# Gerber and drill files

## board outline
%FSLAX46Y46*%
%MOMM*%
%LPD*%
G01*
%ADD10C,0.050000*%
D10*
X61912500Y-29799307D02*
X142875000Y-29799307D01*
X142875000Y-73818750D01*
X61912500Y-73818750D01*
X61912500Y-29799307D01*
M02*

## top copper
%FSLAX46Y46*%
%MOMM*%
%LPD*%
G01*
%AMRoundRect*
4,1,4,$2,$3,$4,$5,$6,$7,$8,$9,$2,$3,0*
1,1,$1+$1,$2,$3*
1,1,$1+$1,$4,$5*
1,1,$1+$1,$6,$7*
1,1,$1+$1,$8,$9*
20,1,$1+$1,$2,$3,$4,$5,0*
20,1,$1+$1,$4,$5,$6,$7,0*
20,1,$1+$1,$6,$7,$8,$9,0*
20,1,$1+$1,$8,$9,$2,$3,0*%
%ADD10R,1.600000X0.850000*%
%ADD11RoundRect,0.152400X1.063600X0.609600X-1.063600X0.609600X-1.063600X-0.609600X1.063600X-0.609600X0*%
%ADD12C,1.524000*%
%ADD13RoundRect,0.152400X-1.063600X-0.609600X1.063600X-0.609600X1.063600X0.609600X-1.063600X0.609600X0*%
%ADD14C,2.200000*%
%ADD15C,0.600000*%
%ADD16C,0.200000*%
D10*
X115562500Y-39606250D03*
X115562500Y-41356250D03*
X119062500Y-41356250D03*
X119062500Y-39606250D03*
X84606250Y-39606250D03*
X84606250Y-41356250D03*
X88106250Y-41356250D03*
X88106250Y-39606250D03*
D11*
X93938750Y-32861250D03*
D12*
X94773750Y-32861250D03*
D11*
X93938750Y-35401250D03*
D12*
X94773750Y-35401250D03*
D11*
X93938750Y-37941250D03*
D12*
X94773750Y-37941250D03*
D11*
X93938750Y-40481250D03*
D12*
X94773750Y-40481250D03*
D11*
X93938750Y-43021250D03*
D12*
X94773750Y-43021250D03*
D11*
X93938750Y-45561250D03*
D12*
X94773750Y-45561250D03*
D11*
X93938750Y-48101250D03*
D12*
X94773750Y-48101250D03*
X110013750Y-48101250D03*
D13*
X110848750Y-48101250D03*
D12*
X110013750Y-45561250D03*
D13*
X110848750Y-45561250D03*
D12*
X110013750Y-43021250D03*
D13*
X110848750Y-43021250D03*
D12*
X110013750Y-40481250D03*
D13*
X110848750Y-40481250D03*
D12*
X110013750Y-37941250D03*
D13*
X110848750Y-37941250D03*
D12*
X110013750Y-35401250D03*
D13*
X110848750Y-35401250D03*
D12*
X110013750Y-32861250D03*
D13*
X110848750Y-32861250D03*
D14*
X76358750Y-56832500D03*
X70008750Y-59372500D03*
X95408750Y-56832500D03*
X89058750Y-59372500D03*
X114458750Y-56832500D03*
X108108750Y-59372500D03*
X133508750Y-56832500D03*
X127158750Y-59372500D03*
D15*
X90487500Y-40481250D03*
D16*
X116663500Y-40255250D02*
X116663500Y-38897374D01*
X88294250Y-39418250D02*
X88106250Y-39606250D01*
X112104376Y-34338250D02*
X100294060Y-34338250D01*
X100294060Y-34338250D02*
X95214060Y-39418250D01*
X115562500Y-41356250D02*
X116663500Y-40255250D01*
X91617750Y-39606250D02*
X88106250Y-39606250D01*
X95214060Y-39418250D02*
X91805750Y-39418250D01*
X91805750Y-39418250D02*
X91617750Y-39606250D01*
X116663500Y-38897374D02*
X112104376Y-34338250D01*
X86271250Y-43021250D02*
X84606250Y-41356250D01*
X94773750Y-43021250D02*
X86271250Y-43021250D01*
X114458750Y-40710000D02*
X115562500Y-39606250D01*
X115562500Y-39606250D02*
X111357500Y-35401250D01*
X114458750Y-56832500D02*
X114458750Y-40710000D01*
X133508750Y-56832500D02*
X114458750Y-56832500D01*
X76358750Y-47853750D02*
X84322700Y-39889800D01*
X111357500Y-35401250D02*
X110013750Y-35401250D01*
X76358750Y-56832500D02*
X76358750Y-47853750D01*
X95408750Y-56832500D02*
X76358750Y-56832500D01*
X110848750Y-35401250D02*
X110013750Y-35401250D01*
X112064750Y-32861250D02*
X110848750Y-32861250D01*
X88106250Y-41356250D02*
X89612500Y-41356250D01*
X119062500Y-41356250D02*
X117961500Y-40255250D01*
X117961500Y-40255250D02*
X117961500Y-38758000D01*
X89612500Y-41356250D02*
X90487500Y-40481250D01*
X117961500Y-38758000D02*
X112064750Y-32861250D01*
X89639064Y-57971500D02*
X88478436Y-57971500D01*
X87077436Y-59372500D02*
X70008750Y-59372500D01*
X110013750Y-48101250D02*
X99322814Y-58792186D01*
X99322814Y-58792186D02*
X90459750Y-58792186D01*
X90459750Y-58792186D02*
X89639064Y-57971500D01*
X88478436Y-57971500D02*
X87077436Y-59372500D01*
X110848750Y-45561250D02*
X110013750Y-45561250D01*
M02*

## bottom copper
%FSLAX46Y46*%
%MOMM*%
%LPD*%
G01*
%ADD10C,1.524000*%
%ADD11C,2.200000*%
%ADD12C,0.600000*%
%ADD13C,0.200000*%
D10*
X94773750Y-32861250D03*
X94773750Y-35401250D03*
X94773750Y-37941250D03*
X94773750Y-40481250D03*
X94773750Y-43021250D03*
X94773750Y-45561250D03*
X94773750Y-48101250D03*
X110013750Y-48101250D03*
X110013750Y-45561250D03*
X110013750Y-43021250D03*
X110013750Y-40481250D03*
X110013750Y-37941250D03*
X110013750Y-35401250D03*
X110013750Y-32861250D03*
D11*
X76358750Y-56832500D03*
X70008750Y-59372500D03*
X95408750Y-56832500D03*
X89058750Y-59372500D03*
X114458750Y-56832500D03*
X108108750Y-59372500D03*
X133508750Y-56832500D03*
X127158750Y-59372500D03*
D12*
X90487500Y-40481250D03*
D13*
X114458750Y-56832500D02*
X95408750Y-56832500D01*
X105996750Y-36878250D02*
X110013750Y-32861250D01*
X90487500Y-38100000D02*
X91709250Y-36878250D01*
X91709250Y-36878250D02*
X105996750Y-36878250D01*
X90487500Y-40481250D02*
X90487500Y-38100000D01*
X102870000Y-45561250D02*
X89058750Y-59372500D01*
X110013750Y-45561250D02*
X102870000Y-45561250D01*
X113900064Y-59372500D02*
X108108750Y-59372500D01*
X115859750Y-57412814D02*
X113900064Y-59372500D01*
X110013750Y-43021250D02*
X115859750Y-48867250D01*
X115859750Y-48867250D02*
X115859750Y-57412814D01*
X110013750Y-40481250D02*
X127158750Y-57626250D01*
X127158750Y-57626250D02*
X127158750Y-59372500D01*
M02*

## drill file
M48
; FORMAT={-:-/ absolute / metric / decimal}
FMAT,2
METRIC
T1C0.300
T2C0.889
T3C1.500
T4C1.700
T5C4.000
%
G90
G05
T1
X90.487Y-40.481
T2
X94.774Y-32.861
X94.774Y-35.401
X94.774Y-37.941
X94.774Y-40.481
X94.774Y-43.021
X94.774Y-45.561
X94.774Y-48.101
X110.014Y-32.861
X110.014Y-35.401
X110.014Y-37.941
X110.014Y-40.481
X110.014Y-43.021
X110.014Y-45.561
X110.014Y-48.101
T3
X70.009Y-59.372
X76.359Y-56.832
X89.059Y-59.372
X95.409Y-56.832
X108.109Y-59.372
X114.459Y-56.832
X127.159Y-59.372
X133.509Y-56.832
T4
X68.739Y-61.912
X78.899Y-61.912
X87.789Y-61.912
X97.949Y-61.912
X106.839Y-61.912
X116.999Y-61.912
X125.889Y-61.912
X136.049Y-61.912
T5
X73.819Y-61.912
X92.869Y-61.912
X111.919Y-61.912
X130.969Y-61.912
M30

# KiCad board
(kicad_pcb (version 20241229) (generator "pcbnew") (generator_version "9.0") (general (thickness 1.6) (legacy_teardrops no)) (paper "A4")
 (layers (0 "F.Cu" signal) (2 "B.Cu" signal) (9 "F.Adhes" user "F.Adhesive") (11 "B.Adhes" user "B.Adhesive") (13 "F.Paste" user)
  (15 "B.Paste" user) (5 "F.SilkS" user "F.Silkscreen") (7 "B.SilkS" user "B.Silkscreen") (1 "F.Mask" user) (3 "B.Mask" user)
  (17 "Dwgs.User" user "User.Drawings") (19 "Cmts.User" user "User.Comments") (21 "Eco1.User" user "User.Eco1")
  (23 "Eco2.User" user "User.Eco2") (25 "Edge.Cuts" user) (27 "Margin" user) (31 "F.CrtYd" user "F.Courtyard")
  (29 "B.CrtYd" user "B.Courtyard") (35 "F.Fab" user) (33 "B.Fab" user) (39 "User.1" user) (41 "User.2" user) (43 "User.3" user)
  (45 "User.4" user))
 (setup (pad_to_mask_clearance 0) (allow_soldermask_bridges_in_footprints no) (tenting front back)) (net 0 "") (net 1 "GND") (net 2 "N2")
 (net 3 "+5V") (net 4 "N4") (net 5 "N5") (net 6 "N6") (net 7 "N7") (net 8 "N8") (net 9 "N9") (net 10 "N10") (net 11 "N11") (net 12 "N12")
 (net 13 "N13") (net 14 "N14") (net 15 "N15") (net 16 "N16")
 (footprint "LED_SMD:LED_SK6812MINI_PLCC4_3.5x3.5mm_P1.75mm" (layer "F.Cu") (at 117.3125 40.48125)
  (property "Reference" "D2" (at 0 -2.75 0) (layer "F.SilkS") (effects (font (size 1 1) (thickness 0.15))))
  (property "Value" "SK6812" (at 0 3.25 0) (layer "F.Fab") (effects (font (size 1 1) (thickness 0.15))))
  (pad "1" smd rect (at -1.75 -0.875) (size 1.6 0.85) (layers "F.Cu" "F.Mask" "F.Paste") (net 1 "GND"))
  (pad "2" smd rect (at -1.75 0.875) (size 1.6 0.85) (layers "F.Cu" "F.Mask" "F.Paste") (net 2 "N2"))
  (pad "3" smd rect (at 1.75 0.875) (size 1.6 0.85) (layers "F.Cu" "F.Mask" "F.Paste") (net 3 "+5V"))
  (pad "4" smd rect (at 1.75 -0.875) (size 1.6 0.85) (layers "F.Cu" "F.Mask" "F.Paste") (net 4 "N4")))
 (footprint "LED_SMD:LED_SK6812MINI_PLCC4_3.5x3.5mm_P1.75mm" (layer "F.Cu") (at 86.35625 40.48125)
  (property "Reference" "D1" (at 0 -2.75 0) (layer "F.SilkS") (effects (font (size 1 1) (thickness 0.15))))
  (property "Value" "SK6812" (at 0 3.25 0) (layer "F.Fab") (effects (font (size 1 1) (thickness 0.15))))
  (pad "1" smd rect (at -1.75 -0.875) (size 1.6 0.85) (layers "F.Cu" "F.Mask" "F.Paste") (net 1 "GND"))
  (pad "2" smd rect (at -1.75 0.875) (size 1.6 0.85) (layers "F.Cu" "F.Mask" "F.Paste") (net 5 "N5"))
  (pad "3" smd rect (at 1.75 0.875) (size 1.6 0.85) (layers "F.Cu" "F.Mask" "F.Paste") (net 3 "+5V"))
  (pad "4" smd rect (at 1.75 -0.875) (size 1.6 0.85) (layers "F.Cu" "F.Mask" "F.Paste") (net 2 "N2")))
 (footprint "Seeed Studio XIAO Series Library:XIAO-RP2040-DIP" (layer "F.Cu") (at 102.39375 40.48125)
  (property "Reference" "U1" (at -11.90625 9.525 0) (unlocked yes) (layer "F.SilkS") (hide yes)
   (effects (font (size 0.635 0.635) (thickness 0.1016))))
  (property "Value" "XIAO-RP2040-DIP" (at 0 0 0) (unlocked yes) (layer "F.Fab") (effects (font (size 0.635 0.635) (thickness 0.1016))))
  (pad "1" smd roundrect (at -8.455 -7.62 180) (size 2.432 1.524) (layers "F.Cu" "F.Mask") (roundrect_rratio 0.1) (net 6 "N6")
   (thermal_bridge_angle 45))
  (pad "1" thru_hole circle (at -7.62 -7.62 180) (size 1.524 1.524) (drill 0.889) (layers "*.Cu" "*.Mask") (remove_unused_layers no)
   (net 6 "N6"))
  (pad "2" smd roundrect (at -8.455 -5.08 180) (size 2.432 1.524) (layers "F.Cu" "F.Mask") (roundrect_rratio 0.1) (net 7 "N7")
   (thermal_bridge_angle 45))
  (pad "2" thru_hole circle (at -7.62 -5.08 180) (size 1.524 1.524) (drill 0.889) (layers "*.Cu" "*.Mask") (remove_unused_layers no)
   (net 7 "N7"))
  (pad "3" smd roundrect (at -8.455 -2.54 180) (size 2.432 1.524) (layers "F.Cu" "F.Mask") (roundrect_rratio 0.1) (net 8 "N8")
   (thermal_bridge_angle 45))
  (pad "3" thru_hole circle (at -7.62 -2.54 180) (size 1.524 1.524) (drill 0.889) (layers "*.Cu" "*.Mask") (remove_unused_layers no)
   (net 8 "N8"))
  (pad "4" smd roundrect (at -8.455 0 180) (size 2.432 1.524) (layers "F.Cu" "F.Mask") (roundrect_rratio 0.1) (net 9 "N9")
   (thermal_bridge_angle 45))
  (pad "4" thru_hole circle (at -7.62 0 180) (size 1.524 1.524) (drill 0.889) (layers "*.Cu" "*.Mask") (remove_unused_layers no)
   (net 9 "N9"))
  (pad "5" smd roundrect (at -8.455 2.54 180) (size 2.432 1.524) (layers "F.Cu" "F.Mask") (roundrect_rratio 0.1) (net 5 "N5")
   (thermal_bridge_angle 45))
  (pad "5" thru_hole circle (at -7.62 2.54 180) (size 1.524 1.524) (drill 0.889) (layers "*.Cu" "*.Mask") (remove_unused_layers no)
   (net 5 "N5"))
  (pad "6" smd roundrect (at -8.455 5.08 180) (size 2.432 1.524) (layers "F.Cu" "F.Mask") (roundrect_rratio 0.1) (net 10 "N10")
   (thermal_bridge_angle 45))
  (pad "6" thru_hole circle (at -7.62 5.08 180) (size 1.524 1.524) (drill 0.889) (layers "*.Cu" "*.Mask") (remove_unused_layers no)
   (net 10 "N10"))
  (pad "7" smd roundrect (at -8.455 7.62 180) (size 2.432 1.524) (layers "F.Cu" "F.Mask") (roundrect_rratio 0.1) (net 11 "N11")
   (thermal_bridge_angle 45))
  (pad "7" thru_hole circle (at -7.62 7.62 180) (size 1.524 1.524) (drill 0.889) (layers "*.Cu" "*.Mask") (remove_unused_layers no)
   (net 11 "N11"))
  (pad "8" thru_hole circle (at 7.62 7.62) (size 1.524 1.524) (drill 0.889) (layers "*.Cu" "*.Mask") (remove_unused_layers no)
   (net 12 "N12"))
  (pad "8" smd roundrect (at 8.455 7.62) (size 2.432 1.524) (layers "F.Cu" "F.Mask") (roundrect_rratio 0.1) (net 12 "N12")
   (thermal_bridge_angle 45))
  (pad "9" thru_hole circle (at 7.62 5.08) (size 1.524 1.524) (drill 0.889) (layers "*.Cu" "*.Mask") (remove_unused_layers no)
   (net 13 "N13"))
  (pad "9" smd roundrect (at 8.455 5.08) (size 2.432 1.524) (layers "F.Cu" "F.Mask") (roundrect_rratio 0.1) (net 13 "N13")
   (thermal_bridge_angle 45))
  (pad "10" thru_hole circle (at 7.62 2.54) (size 1.524 1.524) (drill 0.889) (layers "*.Cu" "*.Mask") (remove_unused_layers no)
   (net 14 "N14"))
  (pad "10" smd roundrect (at 8.455 2.54) (size 2.432 1.524) (layers "F.Cu" "F.Mask") (roundrect_rratio 0.1) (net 14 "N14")
   (thermal_bridge_angle 45))
  (pad "11" thru_hole circle (at 7.62 0) (size 1.524 1.524) (drill 0.889) (layers "*.Cu" "*.Mask") (remove_unused_layers no) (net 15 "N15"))
  (pad "11" smd roundrect (at 8.455 0) (size 2.432 1.524) (layers "F.Cu" "F.Mask") (roundrect_rratio 0.1) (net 15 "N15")
   (thermal_bridge_angle 45))
  (pad "12" thru_hole circle (at 7.62 -2.54) (size 1.524 1.524) (drill 0.889) (layers "*.Cu" "*.Mask") (remove_unused_layers no)
   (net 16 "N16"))
  (pad "12" smd roundrect (at 8.455 -2.54) (size 2.432 1.524) (layers "F.Cu" "F.Mask") (roundrect_rratio 0.1) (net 16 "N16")
   (thermal_bridge_angle 45))
  (pad "13" thru_hole circle (at 7.62 -5.08) (size 1.524 1.524) (drill 0.889) (layers "*.Cu" "*.Mask") (remove_unused_layers no)
   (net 1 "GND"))
  (pad "13" smd roundrect (at 8.455 -5.08) (size 2.432 1.524) (layers "F.Cu" "F.Mask") (roundrect_rratio 0.1) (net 1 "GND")
   (thermal_bridge_angle 45))
  (pad "14" thru_hole circle (at 7.62 -7.62) (size 1.524 1.524) (drill 0.889) (layers "*.Cu" "*.Mask") (remove_unused_layers no)
   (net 3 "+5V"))
  (pad "14" smd roundrect (at 8.455 -7.62) (size 2.432 1.524) (layers "F.Cu" "F.Mask") (roundrect_rratio 0.1) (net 3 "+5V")
   (thermal_bridge_angle 45)))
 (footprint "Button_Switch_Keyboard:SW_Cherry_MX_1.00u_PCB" (layer "F.Cu") (at 76.35875 56.8325)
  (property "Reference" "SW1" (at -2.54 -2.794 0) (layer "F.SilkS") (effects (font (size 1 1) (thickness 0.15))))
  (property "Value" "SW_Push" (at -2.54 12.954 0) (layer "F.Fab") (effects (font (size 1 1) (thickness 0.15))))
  (pad "" np_thru_hole circle (at -7.62 5.08) (size 1.7 1.7) (drill 1.7) (layers "*.Cu" "*.Mask"))
  (pad "" np_thru_hole circle (at -2.54 5.08) (size 4 4) (drill 4) (layers "*.Cu" "*.Mask"))
  (pad "" np_thru_hole circle (at 2.54 5.08) (size 1.7 1.7) (drill 1.7) (layers "*.Cu" "*.Mask"))
  (pad "1" thru_hole circle (at 0 0) (size 2.2 2.2) (drill 1.5) (layers "*.Cu" "*.Mask") (remove_unused_layers no) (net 1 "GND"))
  (pad "2" thru_hole circle (at -6.35 2.54) (size 2.2 2.2) (drill 1.5) (layers "*.Cu" "*.Mask") (remove_unused_layers no) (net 12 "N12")))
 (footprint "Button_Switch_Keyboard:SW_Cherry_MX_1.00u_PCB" (layer "F.Cu") (at 95.40875 56.8325)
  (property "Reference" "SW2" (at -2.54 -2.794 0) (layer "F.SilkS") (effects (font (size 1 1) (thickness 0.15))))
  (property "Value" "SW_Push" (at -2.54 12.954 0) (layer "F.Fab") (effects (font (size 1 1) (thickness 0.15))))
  (pad "" np_thru_hole circle (at -7.62 5.08) (size 1.7 1.7) (drill 1.7) (layers "*.Cu" "*.Mask"))
  (pad "" np_thru_hole circle (at -2.54 5.08) (size 4 4) (drill 4) (layers "*.Cu" "*.Mask"))
  (pad "" np_thru_hole circle (at 2.54 5.08) (size 1.7 1.7) (drill 1.7) (layers "*.Cu" "*.Mask"))
  (pad "1" thru_hole circle (at 0 0) (size 2.2 2.2) (drill 1.5) (layers "*.Cu" "*.Mask") (remove_unused_layers no) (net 1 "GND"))
  (pad "2" thru_hole circle (at -6.35 2.54) (size 2.2 2.2) (drill 1.5) (layers "*.Cu" "*.Mask") (remove_unused_layers no) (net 13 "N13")))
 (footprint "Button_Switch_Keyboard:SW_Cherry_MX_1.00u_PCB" (layer "F.Cu") (at 114.45875 56.8325)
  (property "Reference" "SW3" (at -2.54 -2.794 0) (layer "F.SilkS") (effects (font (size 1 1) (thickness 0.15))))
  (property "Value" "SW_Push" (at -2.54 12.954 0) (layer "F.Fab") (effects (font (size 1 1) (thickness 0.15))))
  (pad "" np_thru_hole circle (at -7.62 5.08) (size 1.7 1.7) (drill 1.7) (layers "*.Cu" "*.Mask"))
  (pad "" np_thru_hole circle (at -2.54 5.08) (size 4 4) (drill 4) (layers "*.Cu" "*.Mask"))
  (pad "" np_thru_hole circle (at 2.54 5.08) (size 1.7 1.7) (drill 1.7) (layers "*.Cu" "*.Mask"))
  (pad "1" thru_hole circle (at 0 0) (size 2.2 2.2) (drill 1.5) (layers "*.Cu" "*.Mask") (remove_unused_layers no) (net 1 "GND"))
  (pad "2" thru_hole circle (at -6.35 2.54) (size 2.2 2.2) (drill 1.5) (layers "*.Cu" "*.Mask") (remove_unused_layers no) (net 14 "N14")))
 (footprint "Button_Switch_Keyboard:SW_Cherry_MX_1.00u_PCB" (layer "F.Cu") (at 133.50875 56.8325)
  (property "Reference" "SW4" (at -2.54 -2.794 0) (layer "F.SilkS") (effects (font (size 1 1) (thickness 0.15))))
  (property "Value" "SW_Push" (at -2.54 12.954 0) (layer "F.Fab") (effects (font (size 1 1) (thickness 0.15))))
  (pad "" np_thru_hole circle (at -7.62 5.08) (size 1.7 1.7) (drill 1.7) (layers "*.Cu" "*.Mask"))
  (pad "" np_thru_hole circle (at -2.54 5.08) (size 4 4) (drill 4) (layers "*.Cu" "*.Mask"))
  (pad "" np_thru_hole circle (at 2.54 5.08) (size 1.7 1.7) (drill 1.7) (layers "*.Cu" "*.Mask"))
  (pad "1" thru_hole circle (at 0 0) (size 2.2 2.2) (drill 1.5) (layers "*.Cu" "*.Mask") (remove_unused_layers no) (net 1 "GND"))
  (pad "2" thru_hole circle (at -6.35 2.54) (size 2.2 2.2) (drill 1.5) (layers "*.Cu" "*.Mask") (remove_unused_layers no) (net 15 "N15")))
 (gr_rect (start 61.9125 29.799307) (end 142.875 73.81875) (stroke (width 0.05) (type default)) (fill no) (layer "Edge.Cuts"))
 (segment (start 116.6635 40.25525) (end 116.6635 38.897374) (width 0.2) (layer "F.Cu") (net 2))
 (segment (start 88.29425 39.41825) (end 88.10625 39.60625) (width 0.2) (layer "F.Cu") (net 2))
 (segment (start 112.104376 34.33825) (end 100.29406 34.33825) (width 0.2) (layer "F.Cu") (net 2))
 (segment (start 100.29406 34.33825) (end 95.21406 39.41825) (width 0.2) (layer "F.Cu") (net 2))
 (segment (start 115.5625 41.35625) (end 116.6635 40.25525) (width 0.2) (layer "F.Cu") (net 2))
 (segment (start 91.61775 39.60625) (end 88.10625 39.60625) (width 0.2) (layer "F.Cu") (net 2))
 (segment (start 95.21406 39.41825) (end 91.80575 39.41825) (width 0.2) (layer "F.Cu") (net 2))
 (segment (start 91.80575 39.41825) (end 91.61775 39.60625) (width 0.2) (layer "F.Cu") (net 2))
 (segment (start 116.6635 38.897374) (end 112.104376 34.33825) (width 0.2) (layer "F.Cu") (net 2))
 (segment (start 86.27125 43.02125) (end 84.60625 41.35625) (width 0.2) (layer "F.Cu") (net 5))
 (segment (start 94.77375 43.02125) (end 86.27125 43.02125) (width 0.2) (layer "F.Cu") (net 5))
 (segment (start 114.45875 40.71) (end 115.5625 39.60625) (width 0.2) (layer "F.Cu") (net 1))
 (segment (start 115.5625 39.60625) (end 111.3575 35.40125) (width 0.2) (layer "F.Cu") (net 1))
 (segment (start 114.45875 56.8325) (end 114.45875 40.71) (width 0.2) (layer "F.Cu") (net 1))
 (segment (start 133.50875 56.8325) (end 114.45875 56.8325) (width 0.2) (layer "F.Cu") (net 1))
 (segment (start 76.35875 47.85375) (end 84.3227 39.8898) (width 0.2) (layer "F.Cu") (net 1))
 (segment (start 111.3575 35.40125) (end 110.01375 35.40125) (width 0.2) (layer "F.Cu") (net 1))
 (segment (start 76.35875 56.8325) (end 76.35875 47.85375) (width 0.2) (layer "F.Cu") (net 1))
 (segment (start 95.40875 56.8325) (end 76.35875 56.8325) (width 0.2) (layer "F.Cu") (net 1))
 (segment (start 110.84875 35.40125) (end 110.01375 35.40125) (width 0.2) (layer "F.Cu") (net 1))
 (segment (start 114.45875 56.8325) (end 95.40875 56.8325) (width 0.2) (layer "B.Cu") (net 1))
 (segment (start 112.06475 32.86125) (end 110.84875 32.86125) (width 0.2) (layer "F.Cu") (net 3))
 (segment (start 88.10625 41.35625) (end 89.6125 41.35625) (width 0.2) (layer "F.Cu") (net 3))
 (segment (start 119.0625 41.35625) (end 117.9615 40.25525) (width 0.2) (layer "F.Cu") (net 3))
 (segment (start 117.9615 40.25525) (end 117.9615 38.758) (width 0.2) (layer "F.Cu") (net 3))
 (segment (start 89.6125 41.35625) (end 90.4875 40.48125) (width 0.2) (layer "F.Cu") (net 3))
 (segment (start 117.9615 38.758) (end 112.06475 32.86125) (width 0.2) (layer "F.Cu") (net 3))
 (via (at 90.4875 40.48125) (size 0.6) (drill 0.3) (layers "F.Cu" "B.Cu") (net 3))
 (segment (start 105.99675 36.87825) (end 110.01375 32.86125) (width 0.2) (layer "B.Cu") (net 3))
 (segment (start 90.4875 38.1) (end 91.70925 36.87825) (width 0.2) (layer "B.Cu") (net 3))
 (segment (start 91.70925 36.87825) (end 105.99675 36.87825) (width 0.2) (layer "B.Cu") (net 3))
 (segment (start 90.4875 40.48125) (end 90.4875 38.1) (width 0.2) (layer "B.Cu") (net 3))
 (segment (start 89.639064 57.9715) (end 88.478436 57.9715) (width 0.2) (layer "F.Cu") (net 12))
 (segment (start 87.077436 59.3725) (end 70.00875 59.3725) (width 0.2) (layer "F.Cu") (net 12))
 (segment (start 110.01375 48.10125) (end 99.322814 58.792186) (width 0.2) (layer "F.Cu") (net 12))
 (segment (start 99.322814 58.792186) (end 90.45975 58.792186) (width 0.2) (layer "F.Cu") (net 12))
 (segment (start 90.45975 58.792186) (end 89.639064 57.9715) (width 0.2) (layer "F.Cu") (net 12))
 (segment (start 88.478436 57.9715) (end 87.077436 59.3725) (width 0.2) (layer "F.Cu") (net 12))
 (segment (start 110.84875 45.56125) (end 110.01375 45.56125) (width 0.2) (layer "F.Cu") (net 13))
 (segment (start 102.87 45.56125) (end 89.05875 59.3725) (width 0.2) (layer "B.Cu") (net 13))
 (segment (start 110.01375 45.56125) (end 102.87 45.56125) (width 0.2) (layer "B.Cu") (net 13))
 (segment (start 113.900064 59.3725) (end 108.10875 59.3725) (width 0.2) (layer "B.Cu") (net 14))
 (segment (start 115.85975 57.412814) (end 113.900064 59.3725) (width 0.2) (layer "B.Cu") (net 14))
 (segment (start 110.01375 43.02125) (end 115.85975 48.86725) (width 0.2) (layer "B.Cu") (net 14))
 (segment (start 115.85975 48.86725) (end 115.85975 57.412814) (width 0.2) (layer "B.Cu") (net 14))
 (segment (start 110.01375 40.48125) (end 127.15875 57.62625) (width 0.2) (layer "B.Cu") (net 15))
 (segment (start 127.15875 57.62625) (end 127.15875 59.3725) (width 0.2) (layer "B.Cu") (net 15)))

